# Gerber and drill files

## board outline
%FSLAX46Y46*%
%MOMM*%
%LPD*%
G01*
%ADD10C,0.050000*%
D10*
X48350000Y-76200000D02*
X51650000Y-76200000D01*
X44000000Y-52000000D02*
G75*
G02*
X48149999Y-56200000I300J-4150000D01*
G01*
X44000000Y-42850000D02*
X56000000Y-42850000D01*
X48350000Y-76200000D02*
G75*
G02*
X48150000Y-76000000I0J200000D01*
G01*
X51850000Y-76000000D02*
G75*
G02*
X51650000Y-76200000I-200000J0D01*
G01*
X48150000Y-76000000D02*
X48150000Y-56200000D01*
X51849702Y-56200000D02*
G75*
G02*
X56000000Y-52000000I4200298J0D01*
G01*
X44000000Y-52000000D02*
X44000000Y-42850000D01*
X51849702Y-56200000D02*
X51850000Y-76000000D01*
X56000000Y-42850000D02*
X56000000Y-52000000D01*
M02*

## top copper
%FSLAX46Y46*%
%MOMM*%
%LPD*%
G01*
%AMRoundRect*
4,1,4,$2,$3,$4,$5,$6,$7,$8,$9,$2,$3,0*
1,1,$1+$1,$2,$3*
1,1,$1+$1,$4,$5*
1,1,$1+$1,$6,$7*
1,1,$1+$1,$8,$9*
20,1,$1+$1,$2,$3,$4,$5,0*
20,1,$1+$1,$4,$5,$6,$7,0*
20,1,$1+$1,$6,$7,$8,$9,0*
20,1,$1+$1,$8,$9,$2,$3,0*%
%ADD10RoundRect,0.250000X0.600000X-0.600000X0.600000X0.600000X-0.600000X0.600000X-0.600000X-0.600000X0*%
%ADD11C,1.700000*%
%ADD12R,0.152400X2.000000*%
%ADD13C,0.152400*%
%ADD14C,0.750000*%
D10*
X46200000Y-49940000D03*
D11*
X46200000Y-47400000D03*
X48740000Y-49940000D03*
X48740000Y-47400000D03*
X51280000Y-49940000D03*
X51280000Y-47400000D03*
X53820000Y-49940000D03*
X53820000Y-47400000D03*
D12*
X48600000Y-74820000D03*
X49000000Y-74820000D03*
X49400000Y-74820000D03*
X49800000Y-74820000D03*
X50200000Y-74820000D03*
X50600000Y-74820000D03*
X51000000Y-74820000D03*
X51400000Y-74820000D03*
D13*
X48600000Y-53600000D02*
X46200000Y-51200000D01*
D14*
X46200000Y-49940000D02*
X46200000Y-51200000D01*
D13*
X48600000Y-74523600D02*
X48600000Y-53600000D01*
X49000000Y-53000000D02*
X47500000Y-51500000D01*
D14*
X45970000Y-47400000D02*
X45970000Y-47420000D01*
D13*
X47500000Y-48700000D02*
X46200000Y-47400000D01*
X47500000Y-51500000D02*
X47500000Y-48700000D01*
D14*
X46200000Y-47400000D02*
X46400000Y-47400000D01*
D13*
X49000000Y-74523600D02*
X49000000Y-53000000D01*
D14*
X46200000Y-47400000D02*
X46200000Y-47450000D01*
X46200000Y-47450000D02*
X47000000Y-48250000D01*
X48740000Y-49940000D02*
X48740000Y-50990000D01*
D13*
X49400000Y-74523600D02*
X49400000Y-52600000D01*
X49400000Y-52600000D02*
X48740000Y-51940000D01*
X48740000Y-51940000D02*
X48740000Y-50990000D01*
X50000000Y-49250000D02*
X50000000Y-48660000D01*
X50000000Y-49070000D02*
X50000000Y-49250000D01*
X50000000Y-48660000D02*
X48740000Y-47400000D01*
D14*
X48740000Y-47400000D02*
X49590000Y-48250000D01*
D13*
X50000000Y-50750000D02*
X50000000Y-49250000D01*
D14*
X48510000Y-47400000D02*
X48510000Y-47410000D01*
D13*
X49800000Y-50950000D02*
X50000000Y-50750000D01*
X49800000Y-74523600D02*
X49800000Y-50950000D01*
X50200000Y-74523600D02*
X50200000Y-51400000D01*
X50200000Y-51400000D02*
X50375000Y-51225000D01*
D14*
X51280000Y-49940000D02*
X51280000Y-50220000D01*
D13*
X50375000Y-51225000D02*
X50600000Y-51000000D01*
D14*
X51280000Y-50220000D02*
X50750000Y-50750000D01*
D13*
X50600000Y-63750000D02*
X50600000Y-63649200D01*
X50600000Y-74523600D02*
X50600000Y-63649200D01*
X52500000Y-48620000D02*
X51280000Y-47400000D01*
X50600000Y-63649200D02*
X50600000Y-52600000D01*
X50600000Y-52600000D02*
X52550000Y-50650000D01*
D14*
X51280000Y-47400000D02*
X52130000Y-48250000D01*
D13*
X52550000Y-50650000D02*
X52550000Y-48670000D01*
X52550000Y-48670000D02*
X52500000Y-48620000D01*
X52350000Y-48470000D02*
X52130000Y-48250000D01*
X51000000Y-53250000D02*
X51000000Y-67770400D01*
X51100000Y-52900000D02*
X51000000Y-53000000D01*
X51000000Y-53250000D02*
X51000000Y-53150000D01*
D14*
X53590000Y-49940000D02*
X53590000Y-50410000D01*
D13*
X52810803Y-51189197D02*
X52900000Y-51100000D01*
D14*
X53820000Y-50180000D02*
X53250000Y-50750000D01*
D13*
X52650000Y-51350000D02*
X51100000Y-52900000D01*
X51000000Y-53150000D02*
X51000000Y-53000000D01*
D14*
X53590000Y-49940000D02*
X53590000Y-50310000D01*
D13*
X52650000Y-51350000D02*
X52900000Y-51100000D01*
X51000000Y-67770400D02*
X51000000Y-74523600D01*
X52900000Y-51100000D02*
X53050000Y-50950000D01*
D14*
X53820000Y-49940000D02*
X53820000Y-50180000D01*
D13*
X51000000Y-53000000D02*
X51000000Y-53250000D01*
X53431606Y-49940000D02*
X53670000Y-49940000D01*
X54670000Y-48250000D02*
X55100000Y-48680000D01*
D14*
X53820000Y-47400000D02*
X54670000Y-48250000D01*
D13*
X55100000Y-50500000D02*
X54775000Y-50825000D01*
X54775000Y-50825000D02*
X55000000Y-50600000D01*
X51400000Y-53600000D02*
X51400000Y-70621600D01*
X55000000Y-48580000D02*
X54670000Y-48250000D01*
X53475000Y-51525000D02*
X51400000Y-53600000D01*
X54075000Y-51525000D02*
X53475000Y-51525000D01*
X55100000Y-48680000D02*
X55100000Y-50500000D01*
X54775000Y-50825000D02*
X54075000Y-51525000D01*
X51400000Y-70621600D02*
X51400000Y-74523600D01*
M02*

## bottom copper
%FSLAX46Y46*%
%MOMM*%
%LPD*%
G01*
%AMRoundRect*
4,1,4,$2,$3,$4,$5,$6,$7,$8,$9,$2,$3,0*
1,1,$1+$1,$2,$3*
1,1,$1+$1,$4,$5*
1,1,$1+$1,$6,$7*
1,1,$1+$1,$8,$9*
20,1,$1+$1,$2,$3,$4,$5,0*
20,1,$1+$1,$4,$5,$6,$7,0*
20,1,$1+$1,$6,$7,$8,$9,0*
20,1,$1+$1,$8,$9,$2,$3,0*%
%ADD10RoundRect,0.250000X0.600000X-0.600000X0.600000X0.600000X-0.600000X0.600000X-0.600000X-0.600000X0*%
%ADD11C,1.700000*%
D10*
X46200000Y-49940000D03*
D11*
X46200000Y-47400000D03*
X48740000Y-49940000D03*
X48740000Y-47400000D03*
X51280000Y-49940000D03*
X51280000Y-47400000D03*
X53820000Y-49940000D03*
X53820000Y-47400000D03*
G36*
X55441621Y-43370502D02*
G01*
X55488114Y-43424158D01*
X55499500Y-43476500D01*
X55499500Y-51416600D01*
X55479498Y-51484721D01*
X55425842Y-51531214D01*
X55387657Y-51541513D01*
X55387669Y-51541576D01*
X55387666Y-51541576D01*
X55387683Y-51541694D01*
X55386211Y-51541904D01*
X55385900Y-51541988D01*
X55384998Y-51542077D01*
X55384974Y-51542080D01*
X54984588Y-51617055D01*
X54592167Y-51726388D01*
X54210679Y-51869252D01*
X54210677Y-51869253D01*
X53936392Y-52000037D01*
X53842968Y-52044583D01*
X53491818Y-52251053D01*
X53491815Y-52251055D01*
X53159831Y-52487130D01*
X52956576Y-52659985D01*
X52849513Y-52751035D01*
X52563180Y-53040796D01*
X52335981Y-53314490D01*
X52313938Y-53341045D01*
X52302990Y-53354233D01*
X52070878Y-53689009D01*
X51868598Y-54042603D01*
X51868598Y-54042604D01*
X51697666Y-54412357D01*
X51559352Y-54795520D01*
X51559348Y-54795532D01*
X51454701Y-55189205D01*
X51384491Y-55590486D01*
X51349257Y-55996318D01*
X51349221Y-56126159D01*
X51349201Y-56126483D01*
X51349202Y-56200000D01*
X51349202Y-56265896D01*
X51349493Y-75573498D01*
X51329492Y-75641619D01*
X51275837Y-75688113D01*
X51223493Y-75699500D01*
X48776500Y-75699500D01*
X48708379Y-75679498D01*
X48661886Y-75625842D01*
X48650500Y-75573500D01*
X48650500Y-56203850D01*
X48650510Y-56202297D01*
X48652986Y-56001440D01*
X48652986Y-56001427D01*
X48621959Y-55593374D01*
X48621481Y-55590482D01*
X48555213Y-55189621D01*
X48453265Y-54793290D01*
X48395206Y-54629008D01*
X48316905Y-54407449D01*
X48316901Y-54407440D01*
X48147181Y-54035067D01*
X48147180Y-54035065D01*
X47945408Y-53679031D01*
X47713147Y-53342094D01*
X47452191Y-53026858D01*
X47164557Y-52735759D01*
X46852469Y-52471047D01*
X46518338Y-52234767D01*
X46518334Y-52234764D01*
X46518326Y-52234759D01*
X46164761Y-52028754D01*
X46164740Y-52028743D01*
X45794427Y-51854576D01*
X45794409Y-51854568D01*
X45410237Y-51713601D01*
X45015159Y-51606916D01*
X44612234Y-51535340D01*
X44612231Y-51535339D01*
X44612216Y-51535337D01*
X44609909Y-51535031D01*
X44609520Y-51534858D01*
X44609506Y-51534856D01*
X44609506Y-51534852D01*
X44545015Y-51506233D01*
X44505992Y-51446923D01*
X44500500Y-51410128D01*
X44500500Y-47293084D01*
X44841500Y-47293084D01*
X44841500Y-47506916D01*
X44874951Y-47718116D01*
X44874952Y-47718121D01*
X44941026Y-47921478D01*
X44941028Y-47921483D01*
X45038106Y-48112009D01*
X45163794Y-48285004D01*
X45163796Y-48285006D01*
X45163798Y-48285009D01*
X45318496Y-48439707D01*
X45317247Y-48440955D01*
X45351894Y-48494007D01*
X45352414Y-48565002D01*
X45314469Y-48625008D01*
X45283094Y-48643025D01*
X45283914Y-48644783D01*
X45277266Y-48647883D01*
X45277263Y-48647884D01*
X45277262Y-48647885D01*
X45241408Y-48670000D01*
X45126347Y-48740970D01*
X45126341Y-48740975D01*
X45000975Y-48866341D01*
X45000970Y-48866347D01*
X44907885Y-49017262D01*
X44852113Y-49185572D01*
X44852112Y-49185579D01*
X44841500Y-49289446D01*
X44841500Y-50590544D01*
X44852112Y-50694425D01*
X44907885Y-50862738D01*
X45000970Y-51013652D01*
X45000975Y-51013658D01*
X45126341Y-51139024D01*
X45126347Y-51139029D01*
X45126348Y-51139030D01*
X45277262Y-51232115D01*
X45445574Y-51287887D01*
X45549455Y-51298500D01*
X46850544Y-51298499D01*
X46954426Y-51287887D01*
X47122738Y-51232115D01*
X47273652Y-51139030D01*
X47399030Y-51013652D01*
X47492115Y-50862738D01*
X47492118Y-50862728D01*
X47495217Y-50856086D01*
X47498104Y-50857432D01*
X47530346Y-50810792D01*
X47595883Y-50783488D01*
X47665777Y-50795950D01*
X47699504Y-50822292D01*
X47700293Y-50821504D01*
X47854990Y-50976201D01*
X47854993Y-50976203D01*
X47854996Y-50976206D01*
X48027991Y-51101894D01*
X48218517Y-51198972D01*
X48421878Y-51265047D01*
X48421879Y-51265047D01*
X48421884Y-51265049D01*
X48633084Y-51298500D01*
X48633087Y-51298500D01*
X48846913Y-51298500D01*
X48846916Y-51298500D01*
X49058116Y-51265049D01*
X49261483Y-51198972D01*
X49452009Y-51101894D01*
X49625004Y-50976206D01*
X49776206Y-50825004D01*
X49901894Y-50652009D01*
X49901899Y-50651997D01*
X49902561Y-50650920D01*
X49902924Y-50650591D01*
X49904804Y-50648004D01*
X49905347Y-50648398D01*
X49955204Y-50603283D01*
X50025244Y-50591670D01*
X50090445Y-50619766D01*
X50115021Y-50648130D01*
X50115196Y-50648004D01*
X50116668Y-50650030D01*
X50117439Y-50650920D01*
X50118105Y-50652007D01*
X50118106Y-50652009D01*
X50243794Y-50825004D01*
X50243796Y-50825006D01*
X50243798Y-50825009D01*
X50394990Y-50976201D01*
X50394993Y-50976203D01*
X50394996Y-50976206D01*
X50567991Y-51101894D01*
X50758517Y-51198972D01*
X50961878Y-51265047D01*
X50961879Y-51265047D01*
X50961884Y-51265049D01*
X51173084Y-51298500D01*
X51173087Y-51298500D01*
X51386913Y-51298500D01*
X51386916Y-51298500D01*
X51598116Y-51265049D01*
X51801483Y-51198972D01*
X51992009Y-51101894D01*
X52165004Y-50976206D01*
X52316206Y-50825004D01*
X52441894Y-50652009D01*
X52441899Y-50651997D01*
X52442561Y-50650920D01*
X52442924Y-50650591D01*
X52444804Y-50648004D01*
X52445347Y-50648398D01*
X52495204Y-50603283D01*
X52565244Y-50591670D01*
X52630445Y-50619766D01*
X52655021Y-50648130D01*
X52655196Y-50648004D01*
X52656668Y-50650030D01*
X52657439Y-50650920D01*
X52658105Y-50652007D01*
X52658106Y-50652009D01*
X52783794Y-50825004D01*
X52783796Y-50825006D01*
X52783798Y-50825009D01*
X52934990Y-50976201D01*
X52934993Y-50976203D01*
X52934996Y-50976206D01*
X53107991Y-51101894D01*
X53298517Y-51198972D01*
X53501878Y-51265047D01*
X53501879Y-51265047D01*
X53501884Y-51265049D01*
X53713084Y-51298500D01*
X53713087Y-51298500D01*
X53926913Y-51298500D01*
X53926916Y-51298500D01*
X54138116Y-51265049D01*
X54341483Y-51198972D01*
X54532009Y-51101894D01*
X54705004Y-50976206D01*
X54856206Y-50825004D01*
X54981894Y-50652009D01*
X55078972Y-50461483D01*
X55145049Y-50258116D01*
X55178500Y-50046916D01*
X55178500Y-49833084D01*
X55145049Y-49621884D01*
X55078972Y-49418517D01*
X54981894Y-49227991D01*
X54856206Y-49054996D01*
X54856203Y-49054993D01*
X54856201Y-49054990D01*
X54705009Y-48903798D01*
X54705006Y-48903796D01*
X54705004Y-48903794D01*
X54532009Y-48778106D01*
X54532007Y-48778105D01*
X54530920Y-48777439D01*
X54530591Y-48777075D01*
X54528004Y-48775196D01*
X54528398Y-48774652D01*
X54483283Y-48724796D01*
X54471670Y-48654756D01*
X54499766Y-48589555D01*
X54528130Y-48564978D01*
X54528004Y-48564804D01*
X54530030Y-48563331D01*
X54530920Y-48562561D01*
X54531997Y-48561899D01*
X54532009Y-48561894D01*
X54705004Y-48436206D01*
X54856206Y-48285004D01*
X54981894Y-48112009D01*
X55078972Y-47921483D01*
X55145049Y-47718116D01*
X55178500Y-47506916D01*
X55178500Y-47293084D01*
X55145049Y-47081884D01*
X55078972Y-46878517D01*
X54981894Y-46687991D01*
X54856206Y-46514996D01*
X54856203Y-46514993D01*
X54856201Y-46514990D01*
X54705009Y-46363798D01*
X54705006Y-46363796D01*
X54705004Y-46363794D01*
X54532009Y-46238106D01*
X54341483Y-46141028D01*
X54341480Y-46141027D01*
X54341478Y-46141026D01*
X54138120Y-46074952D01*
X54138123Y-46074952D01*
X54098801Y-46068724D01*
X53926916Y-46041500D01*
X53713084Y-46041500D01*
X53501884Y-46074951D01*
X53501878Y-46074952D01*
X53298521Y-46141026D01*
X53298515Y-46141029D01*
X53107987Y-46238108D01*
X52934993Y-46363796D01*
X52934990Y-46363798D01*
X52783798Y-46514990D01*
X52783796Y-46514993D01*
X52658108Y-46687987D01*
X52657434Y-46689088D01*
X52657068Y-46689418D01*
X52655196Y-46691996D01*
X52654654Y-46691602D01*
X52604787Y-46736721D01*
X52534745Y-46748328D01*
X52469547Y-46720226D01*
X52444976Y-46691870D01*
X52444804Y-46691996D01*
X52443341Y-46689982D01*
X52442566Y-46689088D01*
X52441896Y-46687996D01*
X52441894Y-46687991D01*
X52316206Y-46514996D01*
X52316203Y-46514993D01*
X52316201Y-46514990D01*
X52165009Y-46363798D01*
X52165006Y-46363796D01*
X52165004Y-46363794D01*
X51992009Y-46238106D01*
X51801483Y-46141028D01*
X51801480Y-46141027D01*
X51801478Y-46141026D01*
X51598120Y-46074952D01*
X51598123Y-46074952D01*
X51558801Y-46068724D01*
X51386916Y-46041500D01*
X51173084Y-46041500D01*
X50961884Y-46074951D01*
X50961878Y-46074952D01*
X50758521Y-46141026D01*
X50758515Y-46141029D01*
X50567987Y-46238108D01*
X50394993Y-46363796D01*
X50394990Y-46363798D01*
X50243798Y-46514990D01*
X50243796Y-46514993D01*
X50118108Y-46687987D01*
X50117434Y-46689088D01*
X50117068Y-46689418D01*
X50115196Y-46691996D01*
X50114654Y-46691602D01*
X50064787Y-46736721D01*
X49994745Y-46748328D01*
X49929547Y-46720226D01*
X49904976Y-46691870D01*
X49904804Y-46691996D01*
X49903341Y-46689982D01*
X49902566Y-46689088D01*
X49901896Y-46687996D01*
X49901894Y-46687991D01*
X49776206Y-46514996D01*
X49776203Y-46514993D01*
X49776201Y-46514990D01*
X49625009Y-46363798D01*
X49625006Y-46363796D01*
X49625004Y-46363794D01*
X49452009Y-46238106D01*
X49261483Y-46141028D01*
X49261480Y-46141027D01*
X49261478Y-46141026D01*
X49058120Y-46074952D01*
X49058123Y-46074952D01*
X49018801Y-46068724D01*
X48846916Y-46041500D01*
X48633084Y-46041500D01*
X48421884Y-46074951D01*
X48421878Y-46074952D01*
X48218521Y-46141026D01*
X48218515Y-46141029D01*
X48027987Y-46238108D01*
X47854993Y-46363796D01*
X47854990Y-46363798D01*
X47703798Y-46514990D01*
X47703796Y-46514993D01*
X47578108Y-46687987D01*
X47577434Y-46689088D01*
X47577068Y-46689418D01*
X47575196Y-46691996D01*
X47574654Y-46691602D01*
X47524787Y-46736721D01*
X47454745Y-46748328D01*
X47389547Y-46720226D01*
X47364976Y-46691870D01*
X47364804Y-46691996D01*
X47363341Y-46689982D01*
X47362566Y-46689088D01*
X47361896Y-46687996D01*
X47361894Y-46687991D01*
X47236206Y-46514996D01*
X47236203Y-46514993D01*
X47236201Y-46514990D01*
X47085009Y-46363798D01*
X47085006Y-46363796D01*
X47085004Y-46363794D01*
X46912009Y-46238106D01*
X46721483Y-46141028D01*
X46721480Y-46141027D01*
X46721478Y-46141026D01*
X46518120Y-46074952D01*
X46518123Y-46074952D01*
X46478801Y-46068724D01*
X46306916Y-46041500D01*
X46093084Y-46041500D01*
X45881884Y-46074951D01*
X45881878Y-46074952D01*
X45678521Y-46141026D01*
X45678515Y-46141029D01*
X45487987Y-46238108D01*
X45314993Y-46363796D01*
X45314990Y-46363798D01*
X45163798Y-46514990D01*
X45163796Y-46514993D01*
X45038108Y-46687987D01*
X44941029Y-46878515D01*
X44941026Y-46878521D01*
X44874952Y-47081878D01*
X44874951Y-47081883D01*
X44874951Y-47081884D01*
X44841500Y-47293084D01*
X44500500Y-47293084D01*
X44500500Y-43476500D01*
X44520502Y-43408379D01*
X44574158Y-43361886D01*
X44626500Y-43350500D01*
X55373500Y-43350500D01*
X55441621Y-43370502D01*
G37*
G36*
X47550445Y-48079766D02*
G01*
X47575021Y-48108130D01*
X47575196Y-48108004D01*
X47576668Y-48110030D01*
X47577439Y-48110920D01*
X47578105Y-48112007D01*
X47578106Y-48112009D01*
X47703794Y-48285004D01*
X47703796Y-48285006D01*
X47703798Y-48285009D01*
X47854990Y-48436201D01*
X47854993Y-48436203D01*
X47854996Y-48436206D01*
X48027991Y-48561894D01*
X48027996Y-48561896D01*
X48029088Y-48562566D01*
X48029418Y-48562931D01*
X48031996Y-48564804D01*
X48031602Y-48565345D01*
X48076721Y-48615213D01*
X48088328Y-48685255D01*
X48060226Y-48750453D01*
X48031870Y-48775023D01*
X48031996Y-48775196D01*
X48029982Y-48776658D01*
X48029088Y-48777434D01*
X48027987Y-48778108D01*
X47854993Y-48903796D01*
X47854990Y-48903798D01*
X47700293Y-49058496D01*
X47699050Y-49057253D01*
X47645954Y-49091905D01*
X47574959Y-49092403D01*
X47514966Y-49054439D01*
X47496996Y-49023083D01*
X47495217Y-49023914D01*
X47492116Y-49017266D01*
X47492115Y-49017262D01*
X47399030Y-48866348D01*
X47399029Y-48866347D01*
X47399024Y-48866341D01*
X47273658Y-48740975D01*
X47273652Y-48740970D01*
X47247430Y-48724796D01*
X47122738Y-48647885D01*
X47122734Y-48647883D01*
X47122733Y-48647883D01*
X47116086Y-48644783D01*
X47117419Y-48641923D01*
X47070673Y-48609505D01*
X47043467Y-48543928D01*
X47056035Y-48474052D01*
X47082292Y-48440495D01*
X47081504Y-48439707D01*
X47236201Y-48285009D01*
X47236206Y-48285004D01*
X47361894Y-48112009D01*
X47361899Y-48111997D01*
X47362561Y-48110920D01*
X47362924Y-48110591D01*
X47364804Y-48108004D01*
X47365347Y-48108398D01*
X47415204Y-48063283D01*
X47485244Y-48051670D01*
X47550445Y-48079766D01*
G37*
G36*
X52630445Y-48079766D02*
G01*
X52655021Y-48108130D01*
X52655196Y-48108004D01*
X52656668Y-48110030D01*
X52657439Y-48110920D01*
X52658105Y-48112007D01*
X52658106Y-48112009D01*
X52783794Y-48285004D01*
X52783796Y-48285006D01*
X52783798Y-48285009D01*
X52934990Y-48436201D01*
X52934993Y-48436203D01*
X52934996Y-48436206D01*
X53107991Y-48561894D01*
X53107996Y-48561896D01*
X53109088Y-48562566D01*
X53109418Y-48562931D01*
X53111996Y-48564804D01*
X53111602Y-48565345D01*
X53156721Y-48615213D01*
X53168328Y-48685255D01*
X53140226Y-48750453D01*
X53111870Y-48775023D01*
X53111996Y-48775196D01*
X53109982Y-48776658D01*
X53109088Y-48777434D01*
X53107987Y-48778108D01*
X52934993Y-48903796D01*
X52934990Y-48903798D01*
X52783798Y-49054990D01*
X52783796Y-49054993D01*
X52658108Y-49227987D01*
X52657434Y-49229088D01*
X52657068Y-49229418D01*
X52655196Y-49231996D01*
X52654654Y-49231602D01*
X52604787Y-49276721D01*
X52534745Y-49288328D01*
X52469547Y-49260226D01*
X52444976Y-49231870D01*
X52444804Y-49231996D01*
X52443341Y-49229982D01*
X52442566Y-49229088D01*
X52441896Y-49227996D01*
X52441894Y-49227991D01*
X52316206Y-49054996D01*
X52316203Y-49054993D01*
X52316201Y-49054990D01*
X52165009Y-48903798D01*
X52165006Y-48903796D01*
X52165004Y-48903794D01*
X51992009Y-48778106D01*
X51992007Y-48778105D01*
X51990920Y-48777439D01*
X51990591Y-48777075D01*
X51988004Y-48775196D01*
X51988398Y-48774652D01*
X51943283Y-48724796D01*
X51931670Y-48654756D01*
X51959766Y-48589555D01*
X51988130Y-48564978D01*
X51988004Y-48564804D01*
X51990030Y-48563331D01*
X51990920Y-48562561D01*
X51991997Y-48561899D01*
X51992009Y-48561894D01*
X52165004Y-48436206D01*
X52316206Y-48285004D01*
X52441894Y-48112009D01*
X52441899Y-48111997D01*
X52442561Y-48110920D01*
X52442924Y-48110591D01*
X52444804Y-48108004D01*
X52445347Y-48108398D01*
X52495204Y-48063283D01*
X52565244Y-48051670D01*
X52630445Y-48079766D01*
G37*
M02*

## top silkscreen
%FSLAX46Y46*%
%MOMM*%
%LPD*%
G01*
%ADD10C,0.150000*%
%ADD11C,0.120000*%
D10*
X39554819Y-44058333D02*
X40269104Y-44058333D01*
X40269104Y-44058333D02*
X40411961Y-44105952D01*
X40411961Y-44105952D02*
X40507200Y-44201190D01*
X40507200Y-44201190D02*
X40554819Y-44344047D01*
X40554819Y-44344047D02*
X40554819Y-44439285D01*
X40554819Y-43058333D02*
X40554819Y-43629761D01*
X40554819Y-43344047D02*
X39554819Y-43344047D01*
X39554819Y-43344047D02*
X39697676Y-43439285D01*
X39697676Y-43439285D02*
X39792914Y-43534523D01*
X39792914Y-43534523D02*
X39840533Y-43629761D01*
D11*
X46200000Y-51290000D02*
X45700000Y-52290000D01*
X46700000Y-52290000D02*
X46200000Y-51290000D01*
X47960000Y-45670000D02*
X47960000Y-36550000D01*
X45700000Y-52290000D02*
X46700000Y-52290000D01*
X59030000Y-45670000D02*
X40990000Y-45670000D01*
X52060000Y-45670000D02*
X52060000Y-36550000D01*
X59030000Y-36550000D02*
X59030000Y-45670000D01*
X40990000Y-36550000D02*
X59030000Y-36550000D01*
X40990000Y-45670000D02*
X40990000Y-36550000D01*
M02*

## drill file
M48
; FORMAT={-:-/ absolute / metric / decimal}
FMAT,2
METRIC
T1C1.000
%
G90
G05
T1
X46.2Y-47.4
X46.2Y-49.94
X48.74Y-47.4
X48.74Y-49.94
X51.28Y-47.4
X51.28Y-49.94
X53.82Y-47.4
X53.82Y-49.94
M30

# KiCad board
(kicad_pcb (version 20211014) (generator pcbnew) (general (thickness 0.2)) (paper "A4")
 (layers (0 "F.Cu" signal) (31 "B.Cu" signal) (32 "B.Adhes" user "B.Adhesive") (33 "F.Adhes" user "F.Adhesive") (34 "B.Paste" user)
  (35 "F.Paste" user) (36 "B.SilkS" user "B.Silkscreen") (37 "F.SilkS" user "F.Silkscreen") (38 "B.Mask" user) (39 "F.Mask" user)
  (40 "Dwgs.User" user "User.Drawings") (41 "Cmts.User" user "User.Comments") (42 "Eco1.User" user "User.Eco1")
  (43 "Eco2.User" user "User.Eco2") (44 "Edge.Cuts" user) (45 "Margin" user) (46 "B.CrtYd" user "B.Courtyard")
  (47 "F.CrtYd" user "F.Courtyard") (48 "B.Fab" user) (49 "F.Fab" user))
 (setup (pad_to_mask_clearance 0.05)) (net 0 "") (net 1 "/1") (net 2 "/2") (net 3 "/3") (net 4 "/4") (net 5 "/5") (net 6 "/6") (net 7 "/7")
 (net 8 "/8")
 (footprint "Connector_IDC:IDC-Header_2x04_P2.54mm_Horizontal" (layer "F.Cu") (at 46.2 49.94 90)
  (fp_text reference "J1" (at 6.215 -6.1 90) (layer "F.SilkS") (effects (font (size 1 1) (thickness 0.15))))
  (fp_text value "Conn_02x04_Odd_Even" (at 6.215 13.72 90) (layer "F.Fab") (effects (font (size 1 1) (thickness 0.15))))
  (fp_line (start -1.35 0) (end -2.35 -0.5) (layer "F.SilkS") (width 0.12))
  (fp_line (start -2.35 0.5) (end -1.35 0) (layer "F.SilkS") (width 0.12))
  (fp_line (start 4.27 1.76) (end 13.39 1.76) (layer "F.SilkS") (width 0.12))
  (fp_line (start -2.35 -0.5) (end -2.35 0.5) (layer "F.SilkS") (width 0.12))
  (fp_line (start 4.27 12.83) (end 4.27 -5.21) (layer "F.SilkS") (width 0.12))
  (fp_line (start 4.27 5.86) (end 13.39 5.86) (layer "F.SilkS") (width 0.12))
  (fp_line (start 13.39 12.83) (end 4.27 12.83) (layer "F.SilkS") (width 0.12))
  (fp_line (start 13.39 -5.21) (end 13.39 12.83) (layer "F.SilkS") (width 0.12))
  (fp_line (start 4.27 -5.21) (end 13.39 -5.21) (layer "F.SilkS") (width 0.12))
  (pad "1" thru_hole roundrect locked (at 0 0 90) (size 1.7 1.7) (drill 1) (layers *.Cu *.Mask) (roundrect_rratio 0.1470588235) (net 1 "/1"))
  (pad "2" thru_hole circle locked (at 2.54 0 90) (size 1.7 1.7) (drill 1) (layers *.Cu *.Mask) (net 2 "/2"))
  (pad "3" thru_hole circle locked (at 0 2.54 90) (size 1.7 1.7) (drill 1) (layers *.Cu *.Mask) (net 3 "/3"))
  (pad "4" thru_hole circle locked (at 2.54 2.54 90) (size 1.7 1.7) (drill 1) (layers *.Cu *.Mask) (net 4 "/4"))
  (pad "5" thru_hole circle locked (at 0 5.08 90) (size 1.7 1.7) (drill 1) (layers *.Cu *.Mask) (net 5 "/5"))
  (pad "6" thru_hole circle locked (at 2.54 5.08 90) (size 1.7 1.7) (drill 1) (layers *.Cu *.Mask) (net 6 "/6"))
  (pad "7" thru_hole circle locked (at 0 7.62 90) (size 1.7 1.7) (drill 1) (layers *.Cu *.Mask) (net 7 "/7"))
  (pad "8" thru_hole circle locked (at 2.54 7.62 90) (size 1.7 1.7) (drill 1) (layers *.Cu *.Mask) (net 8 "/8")))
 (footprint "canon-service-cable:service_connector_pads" (layer "F.Cu") (at 48.25 74.57)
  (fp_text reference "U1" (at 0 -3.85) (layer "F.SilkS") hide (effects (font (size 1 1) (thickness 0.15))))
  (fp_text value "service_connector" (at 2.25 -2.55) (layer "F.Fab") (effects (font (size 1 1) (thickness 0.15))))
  (pad "1" smd rect (at 0.35 0.25) (size 0.1524 2) (layers "F.Cu" "F.Paste" "F.Mask") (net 1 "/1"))
  (pad "2" smd rect (at 0.75 0.25) (size 0.1524 2) (layers "F.Cu" "F.Paste" "F.Mask") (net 2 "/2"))
  (pad "3" smd rect (at 1.15 0.25) (size 0.1524 2) (layers "F.Cu" "F.Paste" "F.Mask") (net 3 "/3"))
  (pad "4" smd rect (at 1.55 0.25) (size 0.1524 2) (layers "F.Cu" "F.Paste" "F.Mask") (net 4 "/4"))
  (pad "5" smd rect (at 1.95 0.25) (size 0.1524 2) (layers "F.Cu" "F.Paste" "F.Mask") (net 5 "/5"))
  (pad "6" smd rect (at 2.35 0.25) (size 0.1524 2) (layers "F.Cu" "F.Paste" "F.Mask") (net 6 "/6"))
  (pad "7" smd rect (at 2.75 0.25) (size 0.1524 2) (layers "F.Cu" "F.Paste" "F.Mask") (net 7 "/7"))
  (pad "8" smd rect (at 3.15 0.25) (size 0.1524 2) (layers "F.Cu" "F.Paste" "F.Mask") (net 8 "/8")))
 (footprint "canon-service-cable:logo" (layer "B.Cu") (at 48.11 54 180)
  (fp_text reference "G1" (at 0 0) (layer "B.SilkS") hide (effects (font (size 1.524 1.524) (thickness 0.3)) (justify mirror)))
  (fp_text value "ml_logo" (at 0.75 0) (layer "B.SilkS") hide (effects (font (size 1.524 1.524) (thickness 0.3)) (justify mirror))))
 (gr_line (start 48.35 76.2) (end 51.65 76.2) (layer "Edge.Cuts") (width 0.05))
 (gr_arc (start 44 52) (mid 46.952314 53.23313) (end 48.15 56.2) (layer "Edge.Cuts") (width 0.05))
 (gr_line (start 44 42.85) (end 56 42.85) (layer "Edge.Cuts") (width 0.05))
 (gr_arc (start 48.35 76.2) (mid 48.208579 76.141421) (end 48.15 76) (layer "Edge.Cuts") (width 0.05))
 (gr_arc (start 51.85 76) (mid 51.791421 76.141421) (end 51.65 76.2) (layer "Edge.Cuts") (width 0.05))
 (gr_line (start 48.15 76) (end 48.15 56.2) (layer "Edge.Cuts") (width 0.05))
 (gr_arc (start 51.849702 56.2) (mid 53.062315 53.247671) (end 56 52) (layer "Edge.Cuts") (width 0.05))
 (gr_line (start 44 52) (end 44 42.85) (layer "Edge.Cuts") (width 0.05))
 (gr_line (start 51.849702 56.2) (end 51.85 76) (layer "Edge.Cuts") (width 0.05))
 (gr_line (start 56 42.85) (end 56 52) (layer "Edge.Cuts") (width 0.05))
 (segment (start 48.6 53.6) (end 46.2 51.2) (width 0.1524) (layer "F.Cu") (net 1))
 (segment (start 46.2 49.94) (end 46.2 51.2) (width 0.75) (layer "F.Cu") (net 1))
 (segment (start 48.6 74.5236) (end 48.6 53.6) (width 0.1524) (layer "F.Cu") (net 1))
 (segment (start 49 53) (end 47.5 51.5) (width 0.1524) (layer "F.Cu") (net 2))
 (segment (start 45.97 47.4) (end 45.97 47.42) (width 0.75) (layer "F.Cu") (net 2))
 (segment (start 47.5 48.7) (end 46.2 47.4) (width 0.1524) (layer "F.Cu") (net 2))
 (segment (start 47.5 51.5) (end 47.5 48.7) (width 0.1524) (layer "F.Cu") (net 2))
 (segment (start 46.2 47.4) (end 46.4 47.4) (width 0.75) (layer "F.Cu") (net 2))
 (segment (start 49 74.5236) (end 49 53) (width 0.1524) (layer "F.Cu") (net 2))
 (segment (start 46.2 47.4) (end 46.2 47.45) (width 0.75) (layer "F.Cu") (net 2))
 (segment (start 46.2 47.45) (end 47 48.25) (width 0.75) (layer "F.Cu") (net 2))
 (segment (start 48.74 49.94) (end 48.74 50.99) (width 0.75) (layer "F.Cu") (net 3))
 (segment (start 49.4 74.5236) (end 49.4 52.6) (width 0.1524) (layer "F.Cu") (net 3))
 (segment (start 49.4 52.6) (end 48.74 51.94) (width 0.1524) (layer "F.Cu") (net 3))
 (segment (start 48.74 51.94) (end 48.74 50.99) (width 0.1524) (layer "F.Cu") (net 3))
 (segment (start 50 49.25) (end 50 48.66) (width 0.1524) (layer "F.Cu") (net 4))
 (segment (start 50 49.07) (end 50 49.25) (width 0.1524) (layer "F.Cu") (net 4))
 (segment (start 50 48.66) (end 48.74 47.4) (width 0.1524) (layer "F.Cu") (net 4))
 (segment (start 48.74 47.4) (end 49.59 48.25) (width 0.75) (layer "F.Cu") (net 4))
 (segment (start 50 50.75) (end 50 49.25) (width 0.1524) (layer "F.Cu") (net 4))
 (segment (start 48.51 47.4) (end 48.51 47.41) (width 0.75) (layer "F.Cu") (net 4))
 (segment (start 49.8 50.95) (end 50 50.75) (width 0.1524) (layer "F.Cu") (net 4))
 (segment (start 49.8 74.5236) (end 49.8 50.95) (width 0.1524) (layer "F.Cu") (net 4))
 (segment (start 50.2 74.5236) (end 50.2 51.4) (width 0.1524) (layer "F.Cu") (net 5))
 (segment (start 50.2 51.4) (end 50.375 51.225) (width 0.1524) (layer "F.Cu") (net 5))
 (segment (start 51.28 49.94) (end 51.28 50.22) (width 0.75) (layer "F.Cu") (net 5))
 (segment (start 50.375 51.225) (end 50.6 51) (width 0.1524) (layer "F.Cu") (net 5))
 (segment (start 51.28 50.22) (end 50.75 50.75) (width 0.75) (layer "F.Cu") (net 5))
 (segment (start 50.6 63.75) (end 50.6 63.6492) (width 0.1524) (layer "F.Cu") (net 6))
 (segment (start 50.6 74.5236) (end 50.6 63.6492) (width 0.1524) (layer "F.Cu") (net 6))
 (segment (start 52.5 48.62) (end 51.28 47.4) (width 0.1524) (layer "F.Cu") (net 6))
 (segment (start 50.6 63.6492) (end 50.6 52.6) (width 0.1524) (layer "F.Cu") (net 6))
 (segment (start 50.6 52.6) (end 52.55 50.65) (width 0.1524) (layer "F.Cu") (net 6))
 (segment (start 51.28 47.4) (end 52.13 48.25) (width 0.75) (layer "F.Cu") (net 6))
 (segment (start 52.55 50.65) (end 52.55 48.67) (width 0.1524) (layer "F.Cu") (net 6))
 (segment (start 52.55 48.67) (end 52.5 48.62) (width 0.1524) (layer "F.Cu") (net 6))
 (segment (start 52.35 48.47) (end 52.13 48.25) (width 0.1524) (layer "F.Cu") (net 6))
 (segment (start 51 53.25) (end 51 67.7704) (width 0.1524) (layer "F.Cu") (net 7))
 (segment (start 51.1 52.9) (end 51 53) (width 0.1524) (layer "F.Cu") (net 7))
 (segment (start 51 53.25) (end 51 53.15) (width 0.1524) (layer "F.Cu") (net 7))
 (segment (start 53.59 49.94) (end 53.59 50.41) (width 0.75) (layer "F.Cu") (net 7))
 (segment (start 52.810803 51.189197) (end 52.9 51.1) (width 0.1524) (layer "F.Cu") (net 7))
 (segment (start 53.82 50.18) (end 53.25 50.75) (width 0.75) (layer "F.Cu") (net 7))
 (segment (start 52.65 51.35) (end 51.1 52.9) (width 0.1524) (layer "F.Cu") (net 7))
 (segment (start 51 53.15) (end 51 53) (width 0.1524) (layer "F.Cu") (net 7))
 (segment (start 53.59 49.94) (end 53.59 50.31) (width 0.75) (layer "F.Cu") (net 7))
 (segment (start 52.65 51.35) (end 52.9 51.1) (width 0.1524) (layer "F.Cu") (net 7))
 (segment (start 51 67.7704) (end 51 74.5236) (width 0.1524) (layer "F.Cu") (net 7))
 (segment (start 52.9 51.1) (end 53.05 50.95) (width 0.1524) (layer "F.Cu") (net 7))
 (segment (start 53.82 49.94) (end 53.82 50.18) (width 0.75) (layer "F.Cu") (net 7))
 (segment (start 51 53) (end 51 53.25) (width 0.1524) (layer "F.Cu") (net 7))
 (segment (start 53.431606 49.94) (end 53.67 49.94) (width 0.1524) (layer "F.Cu") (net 7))
 (segment (start 54.67 48.25) (end 55.1 48.68) (width 0.1524) (layer "F.Cu") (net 8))
 (segment (start 53.82 47.4) (end 54.67 48.25) (width 0.75) (layer "F.Cu") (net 8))
 (segment (start 55.1 50.5) (end 54.775 50.825) (width 0.1524) (layer "F.Cu") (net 8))
 (segment (start 54.775 50.825) (end 55 50.6) (width 0.1524) (layer "F.Cu") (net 8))
 (segment (start 51.4 53.6) (end 51.4 70.6216) (width 0.1524) (layer "F.Cu") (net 8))
 (segment (start 55 48.58) (end 54.67 48.25) (width 0.1524) (layer "F.Cu") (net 8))
 (segment (start 53.475 51.525) (end 51.4 53.6) (width 0.1524) (layer "F.Cu") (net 8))
 (segment (start 54.075 51.525) (end 53.475 51.525) (width 0.1524) (layer "F.Cu") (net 8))
 (segment (start 55.1 48.68) (end 55.1 50.5) (width 0.1524) (layer "F.Cu") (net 8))
 (segment (start 54.775 50.825) (end 54.075 51.525) (width 0.1524) (layer "F.Cu") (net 8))
 (segment (start 51.4 70.6216) (end 51.4 74.5236) (width 0.1524) (layer "F.Cu") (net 8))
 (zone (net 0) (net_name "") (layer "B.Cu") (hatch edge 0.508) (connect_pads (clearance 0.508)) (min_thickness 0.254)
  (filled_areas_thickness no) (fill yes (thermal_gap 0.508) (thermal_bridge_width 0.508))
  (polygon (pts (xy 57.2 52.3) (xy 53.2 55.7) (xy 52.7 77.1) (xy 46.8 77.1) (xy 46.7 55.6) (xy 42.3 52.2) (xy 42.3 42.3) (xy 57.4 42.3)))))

